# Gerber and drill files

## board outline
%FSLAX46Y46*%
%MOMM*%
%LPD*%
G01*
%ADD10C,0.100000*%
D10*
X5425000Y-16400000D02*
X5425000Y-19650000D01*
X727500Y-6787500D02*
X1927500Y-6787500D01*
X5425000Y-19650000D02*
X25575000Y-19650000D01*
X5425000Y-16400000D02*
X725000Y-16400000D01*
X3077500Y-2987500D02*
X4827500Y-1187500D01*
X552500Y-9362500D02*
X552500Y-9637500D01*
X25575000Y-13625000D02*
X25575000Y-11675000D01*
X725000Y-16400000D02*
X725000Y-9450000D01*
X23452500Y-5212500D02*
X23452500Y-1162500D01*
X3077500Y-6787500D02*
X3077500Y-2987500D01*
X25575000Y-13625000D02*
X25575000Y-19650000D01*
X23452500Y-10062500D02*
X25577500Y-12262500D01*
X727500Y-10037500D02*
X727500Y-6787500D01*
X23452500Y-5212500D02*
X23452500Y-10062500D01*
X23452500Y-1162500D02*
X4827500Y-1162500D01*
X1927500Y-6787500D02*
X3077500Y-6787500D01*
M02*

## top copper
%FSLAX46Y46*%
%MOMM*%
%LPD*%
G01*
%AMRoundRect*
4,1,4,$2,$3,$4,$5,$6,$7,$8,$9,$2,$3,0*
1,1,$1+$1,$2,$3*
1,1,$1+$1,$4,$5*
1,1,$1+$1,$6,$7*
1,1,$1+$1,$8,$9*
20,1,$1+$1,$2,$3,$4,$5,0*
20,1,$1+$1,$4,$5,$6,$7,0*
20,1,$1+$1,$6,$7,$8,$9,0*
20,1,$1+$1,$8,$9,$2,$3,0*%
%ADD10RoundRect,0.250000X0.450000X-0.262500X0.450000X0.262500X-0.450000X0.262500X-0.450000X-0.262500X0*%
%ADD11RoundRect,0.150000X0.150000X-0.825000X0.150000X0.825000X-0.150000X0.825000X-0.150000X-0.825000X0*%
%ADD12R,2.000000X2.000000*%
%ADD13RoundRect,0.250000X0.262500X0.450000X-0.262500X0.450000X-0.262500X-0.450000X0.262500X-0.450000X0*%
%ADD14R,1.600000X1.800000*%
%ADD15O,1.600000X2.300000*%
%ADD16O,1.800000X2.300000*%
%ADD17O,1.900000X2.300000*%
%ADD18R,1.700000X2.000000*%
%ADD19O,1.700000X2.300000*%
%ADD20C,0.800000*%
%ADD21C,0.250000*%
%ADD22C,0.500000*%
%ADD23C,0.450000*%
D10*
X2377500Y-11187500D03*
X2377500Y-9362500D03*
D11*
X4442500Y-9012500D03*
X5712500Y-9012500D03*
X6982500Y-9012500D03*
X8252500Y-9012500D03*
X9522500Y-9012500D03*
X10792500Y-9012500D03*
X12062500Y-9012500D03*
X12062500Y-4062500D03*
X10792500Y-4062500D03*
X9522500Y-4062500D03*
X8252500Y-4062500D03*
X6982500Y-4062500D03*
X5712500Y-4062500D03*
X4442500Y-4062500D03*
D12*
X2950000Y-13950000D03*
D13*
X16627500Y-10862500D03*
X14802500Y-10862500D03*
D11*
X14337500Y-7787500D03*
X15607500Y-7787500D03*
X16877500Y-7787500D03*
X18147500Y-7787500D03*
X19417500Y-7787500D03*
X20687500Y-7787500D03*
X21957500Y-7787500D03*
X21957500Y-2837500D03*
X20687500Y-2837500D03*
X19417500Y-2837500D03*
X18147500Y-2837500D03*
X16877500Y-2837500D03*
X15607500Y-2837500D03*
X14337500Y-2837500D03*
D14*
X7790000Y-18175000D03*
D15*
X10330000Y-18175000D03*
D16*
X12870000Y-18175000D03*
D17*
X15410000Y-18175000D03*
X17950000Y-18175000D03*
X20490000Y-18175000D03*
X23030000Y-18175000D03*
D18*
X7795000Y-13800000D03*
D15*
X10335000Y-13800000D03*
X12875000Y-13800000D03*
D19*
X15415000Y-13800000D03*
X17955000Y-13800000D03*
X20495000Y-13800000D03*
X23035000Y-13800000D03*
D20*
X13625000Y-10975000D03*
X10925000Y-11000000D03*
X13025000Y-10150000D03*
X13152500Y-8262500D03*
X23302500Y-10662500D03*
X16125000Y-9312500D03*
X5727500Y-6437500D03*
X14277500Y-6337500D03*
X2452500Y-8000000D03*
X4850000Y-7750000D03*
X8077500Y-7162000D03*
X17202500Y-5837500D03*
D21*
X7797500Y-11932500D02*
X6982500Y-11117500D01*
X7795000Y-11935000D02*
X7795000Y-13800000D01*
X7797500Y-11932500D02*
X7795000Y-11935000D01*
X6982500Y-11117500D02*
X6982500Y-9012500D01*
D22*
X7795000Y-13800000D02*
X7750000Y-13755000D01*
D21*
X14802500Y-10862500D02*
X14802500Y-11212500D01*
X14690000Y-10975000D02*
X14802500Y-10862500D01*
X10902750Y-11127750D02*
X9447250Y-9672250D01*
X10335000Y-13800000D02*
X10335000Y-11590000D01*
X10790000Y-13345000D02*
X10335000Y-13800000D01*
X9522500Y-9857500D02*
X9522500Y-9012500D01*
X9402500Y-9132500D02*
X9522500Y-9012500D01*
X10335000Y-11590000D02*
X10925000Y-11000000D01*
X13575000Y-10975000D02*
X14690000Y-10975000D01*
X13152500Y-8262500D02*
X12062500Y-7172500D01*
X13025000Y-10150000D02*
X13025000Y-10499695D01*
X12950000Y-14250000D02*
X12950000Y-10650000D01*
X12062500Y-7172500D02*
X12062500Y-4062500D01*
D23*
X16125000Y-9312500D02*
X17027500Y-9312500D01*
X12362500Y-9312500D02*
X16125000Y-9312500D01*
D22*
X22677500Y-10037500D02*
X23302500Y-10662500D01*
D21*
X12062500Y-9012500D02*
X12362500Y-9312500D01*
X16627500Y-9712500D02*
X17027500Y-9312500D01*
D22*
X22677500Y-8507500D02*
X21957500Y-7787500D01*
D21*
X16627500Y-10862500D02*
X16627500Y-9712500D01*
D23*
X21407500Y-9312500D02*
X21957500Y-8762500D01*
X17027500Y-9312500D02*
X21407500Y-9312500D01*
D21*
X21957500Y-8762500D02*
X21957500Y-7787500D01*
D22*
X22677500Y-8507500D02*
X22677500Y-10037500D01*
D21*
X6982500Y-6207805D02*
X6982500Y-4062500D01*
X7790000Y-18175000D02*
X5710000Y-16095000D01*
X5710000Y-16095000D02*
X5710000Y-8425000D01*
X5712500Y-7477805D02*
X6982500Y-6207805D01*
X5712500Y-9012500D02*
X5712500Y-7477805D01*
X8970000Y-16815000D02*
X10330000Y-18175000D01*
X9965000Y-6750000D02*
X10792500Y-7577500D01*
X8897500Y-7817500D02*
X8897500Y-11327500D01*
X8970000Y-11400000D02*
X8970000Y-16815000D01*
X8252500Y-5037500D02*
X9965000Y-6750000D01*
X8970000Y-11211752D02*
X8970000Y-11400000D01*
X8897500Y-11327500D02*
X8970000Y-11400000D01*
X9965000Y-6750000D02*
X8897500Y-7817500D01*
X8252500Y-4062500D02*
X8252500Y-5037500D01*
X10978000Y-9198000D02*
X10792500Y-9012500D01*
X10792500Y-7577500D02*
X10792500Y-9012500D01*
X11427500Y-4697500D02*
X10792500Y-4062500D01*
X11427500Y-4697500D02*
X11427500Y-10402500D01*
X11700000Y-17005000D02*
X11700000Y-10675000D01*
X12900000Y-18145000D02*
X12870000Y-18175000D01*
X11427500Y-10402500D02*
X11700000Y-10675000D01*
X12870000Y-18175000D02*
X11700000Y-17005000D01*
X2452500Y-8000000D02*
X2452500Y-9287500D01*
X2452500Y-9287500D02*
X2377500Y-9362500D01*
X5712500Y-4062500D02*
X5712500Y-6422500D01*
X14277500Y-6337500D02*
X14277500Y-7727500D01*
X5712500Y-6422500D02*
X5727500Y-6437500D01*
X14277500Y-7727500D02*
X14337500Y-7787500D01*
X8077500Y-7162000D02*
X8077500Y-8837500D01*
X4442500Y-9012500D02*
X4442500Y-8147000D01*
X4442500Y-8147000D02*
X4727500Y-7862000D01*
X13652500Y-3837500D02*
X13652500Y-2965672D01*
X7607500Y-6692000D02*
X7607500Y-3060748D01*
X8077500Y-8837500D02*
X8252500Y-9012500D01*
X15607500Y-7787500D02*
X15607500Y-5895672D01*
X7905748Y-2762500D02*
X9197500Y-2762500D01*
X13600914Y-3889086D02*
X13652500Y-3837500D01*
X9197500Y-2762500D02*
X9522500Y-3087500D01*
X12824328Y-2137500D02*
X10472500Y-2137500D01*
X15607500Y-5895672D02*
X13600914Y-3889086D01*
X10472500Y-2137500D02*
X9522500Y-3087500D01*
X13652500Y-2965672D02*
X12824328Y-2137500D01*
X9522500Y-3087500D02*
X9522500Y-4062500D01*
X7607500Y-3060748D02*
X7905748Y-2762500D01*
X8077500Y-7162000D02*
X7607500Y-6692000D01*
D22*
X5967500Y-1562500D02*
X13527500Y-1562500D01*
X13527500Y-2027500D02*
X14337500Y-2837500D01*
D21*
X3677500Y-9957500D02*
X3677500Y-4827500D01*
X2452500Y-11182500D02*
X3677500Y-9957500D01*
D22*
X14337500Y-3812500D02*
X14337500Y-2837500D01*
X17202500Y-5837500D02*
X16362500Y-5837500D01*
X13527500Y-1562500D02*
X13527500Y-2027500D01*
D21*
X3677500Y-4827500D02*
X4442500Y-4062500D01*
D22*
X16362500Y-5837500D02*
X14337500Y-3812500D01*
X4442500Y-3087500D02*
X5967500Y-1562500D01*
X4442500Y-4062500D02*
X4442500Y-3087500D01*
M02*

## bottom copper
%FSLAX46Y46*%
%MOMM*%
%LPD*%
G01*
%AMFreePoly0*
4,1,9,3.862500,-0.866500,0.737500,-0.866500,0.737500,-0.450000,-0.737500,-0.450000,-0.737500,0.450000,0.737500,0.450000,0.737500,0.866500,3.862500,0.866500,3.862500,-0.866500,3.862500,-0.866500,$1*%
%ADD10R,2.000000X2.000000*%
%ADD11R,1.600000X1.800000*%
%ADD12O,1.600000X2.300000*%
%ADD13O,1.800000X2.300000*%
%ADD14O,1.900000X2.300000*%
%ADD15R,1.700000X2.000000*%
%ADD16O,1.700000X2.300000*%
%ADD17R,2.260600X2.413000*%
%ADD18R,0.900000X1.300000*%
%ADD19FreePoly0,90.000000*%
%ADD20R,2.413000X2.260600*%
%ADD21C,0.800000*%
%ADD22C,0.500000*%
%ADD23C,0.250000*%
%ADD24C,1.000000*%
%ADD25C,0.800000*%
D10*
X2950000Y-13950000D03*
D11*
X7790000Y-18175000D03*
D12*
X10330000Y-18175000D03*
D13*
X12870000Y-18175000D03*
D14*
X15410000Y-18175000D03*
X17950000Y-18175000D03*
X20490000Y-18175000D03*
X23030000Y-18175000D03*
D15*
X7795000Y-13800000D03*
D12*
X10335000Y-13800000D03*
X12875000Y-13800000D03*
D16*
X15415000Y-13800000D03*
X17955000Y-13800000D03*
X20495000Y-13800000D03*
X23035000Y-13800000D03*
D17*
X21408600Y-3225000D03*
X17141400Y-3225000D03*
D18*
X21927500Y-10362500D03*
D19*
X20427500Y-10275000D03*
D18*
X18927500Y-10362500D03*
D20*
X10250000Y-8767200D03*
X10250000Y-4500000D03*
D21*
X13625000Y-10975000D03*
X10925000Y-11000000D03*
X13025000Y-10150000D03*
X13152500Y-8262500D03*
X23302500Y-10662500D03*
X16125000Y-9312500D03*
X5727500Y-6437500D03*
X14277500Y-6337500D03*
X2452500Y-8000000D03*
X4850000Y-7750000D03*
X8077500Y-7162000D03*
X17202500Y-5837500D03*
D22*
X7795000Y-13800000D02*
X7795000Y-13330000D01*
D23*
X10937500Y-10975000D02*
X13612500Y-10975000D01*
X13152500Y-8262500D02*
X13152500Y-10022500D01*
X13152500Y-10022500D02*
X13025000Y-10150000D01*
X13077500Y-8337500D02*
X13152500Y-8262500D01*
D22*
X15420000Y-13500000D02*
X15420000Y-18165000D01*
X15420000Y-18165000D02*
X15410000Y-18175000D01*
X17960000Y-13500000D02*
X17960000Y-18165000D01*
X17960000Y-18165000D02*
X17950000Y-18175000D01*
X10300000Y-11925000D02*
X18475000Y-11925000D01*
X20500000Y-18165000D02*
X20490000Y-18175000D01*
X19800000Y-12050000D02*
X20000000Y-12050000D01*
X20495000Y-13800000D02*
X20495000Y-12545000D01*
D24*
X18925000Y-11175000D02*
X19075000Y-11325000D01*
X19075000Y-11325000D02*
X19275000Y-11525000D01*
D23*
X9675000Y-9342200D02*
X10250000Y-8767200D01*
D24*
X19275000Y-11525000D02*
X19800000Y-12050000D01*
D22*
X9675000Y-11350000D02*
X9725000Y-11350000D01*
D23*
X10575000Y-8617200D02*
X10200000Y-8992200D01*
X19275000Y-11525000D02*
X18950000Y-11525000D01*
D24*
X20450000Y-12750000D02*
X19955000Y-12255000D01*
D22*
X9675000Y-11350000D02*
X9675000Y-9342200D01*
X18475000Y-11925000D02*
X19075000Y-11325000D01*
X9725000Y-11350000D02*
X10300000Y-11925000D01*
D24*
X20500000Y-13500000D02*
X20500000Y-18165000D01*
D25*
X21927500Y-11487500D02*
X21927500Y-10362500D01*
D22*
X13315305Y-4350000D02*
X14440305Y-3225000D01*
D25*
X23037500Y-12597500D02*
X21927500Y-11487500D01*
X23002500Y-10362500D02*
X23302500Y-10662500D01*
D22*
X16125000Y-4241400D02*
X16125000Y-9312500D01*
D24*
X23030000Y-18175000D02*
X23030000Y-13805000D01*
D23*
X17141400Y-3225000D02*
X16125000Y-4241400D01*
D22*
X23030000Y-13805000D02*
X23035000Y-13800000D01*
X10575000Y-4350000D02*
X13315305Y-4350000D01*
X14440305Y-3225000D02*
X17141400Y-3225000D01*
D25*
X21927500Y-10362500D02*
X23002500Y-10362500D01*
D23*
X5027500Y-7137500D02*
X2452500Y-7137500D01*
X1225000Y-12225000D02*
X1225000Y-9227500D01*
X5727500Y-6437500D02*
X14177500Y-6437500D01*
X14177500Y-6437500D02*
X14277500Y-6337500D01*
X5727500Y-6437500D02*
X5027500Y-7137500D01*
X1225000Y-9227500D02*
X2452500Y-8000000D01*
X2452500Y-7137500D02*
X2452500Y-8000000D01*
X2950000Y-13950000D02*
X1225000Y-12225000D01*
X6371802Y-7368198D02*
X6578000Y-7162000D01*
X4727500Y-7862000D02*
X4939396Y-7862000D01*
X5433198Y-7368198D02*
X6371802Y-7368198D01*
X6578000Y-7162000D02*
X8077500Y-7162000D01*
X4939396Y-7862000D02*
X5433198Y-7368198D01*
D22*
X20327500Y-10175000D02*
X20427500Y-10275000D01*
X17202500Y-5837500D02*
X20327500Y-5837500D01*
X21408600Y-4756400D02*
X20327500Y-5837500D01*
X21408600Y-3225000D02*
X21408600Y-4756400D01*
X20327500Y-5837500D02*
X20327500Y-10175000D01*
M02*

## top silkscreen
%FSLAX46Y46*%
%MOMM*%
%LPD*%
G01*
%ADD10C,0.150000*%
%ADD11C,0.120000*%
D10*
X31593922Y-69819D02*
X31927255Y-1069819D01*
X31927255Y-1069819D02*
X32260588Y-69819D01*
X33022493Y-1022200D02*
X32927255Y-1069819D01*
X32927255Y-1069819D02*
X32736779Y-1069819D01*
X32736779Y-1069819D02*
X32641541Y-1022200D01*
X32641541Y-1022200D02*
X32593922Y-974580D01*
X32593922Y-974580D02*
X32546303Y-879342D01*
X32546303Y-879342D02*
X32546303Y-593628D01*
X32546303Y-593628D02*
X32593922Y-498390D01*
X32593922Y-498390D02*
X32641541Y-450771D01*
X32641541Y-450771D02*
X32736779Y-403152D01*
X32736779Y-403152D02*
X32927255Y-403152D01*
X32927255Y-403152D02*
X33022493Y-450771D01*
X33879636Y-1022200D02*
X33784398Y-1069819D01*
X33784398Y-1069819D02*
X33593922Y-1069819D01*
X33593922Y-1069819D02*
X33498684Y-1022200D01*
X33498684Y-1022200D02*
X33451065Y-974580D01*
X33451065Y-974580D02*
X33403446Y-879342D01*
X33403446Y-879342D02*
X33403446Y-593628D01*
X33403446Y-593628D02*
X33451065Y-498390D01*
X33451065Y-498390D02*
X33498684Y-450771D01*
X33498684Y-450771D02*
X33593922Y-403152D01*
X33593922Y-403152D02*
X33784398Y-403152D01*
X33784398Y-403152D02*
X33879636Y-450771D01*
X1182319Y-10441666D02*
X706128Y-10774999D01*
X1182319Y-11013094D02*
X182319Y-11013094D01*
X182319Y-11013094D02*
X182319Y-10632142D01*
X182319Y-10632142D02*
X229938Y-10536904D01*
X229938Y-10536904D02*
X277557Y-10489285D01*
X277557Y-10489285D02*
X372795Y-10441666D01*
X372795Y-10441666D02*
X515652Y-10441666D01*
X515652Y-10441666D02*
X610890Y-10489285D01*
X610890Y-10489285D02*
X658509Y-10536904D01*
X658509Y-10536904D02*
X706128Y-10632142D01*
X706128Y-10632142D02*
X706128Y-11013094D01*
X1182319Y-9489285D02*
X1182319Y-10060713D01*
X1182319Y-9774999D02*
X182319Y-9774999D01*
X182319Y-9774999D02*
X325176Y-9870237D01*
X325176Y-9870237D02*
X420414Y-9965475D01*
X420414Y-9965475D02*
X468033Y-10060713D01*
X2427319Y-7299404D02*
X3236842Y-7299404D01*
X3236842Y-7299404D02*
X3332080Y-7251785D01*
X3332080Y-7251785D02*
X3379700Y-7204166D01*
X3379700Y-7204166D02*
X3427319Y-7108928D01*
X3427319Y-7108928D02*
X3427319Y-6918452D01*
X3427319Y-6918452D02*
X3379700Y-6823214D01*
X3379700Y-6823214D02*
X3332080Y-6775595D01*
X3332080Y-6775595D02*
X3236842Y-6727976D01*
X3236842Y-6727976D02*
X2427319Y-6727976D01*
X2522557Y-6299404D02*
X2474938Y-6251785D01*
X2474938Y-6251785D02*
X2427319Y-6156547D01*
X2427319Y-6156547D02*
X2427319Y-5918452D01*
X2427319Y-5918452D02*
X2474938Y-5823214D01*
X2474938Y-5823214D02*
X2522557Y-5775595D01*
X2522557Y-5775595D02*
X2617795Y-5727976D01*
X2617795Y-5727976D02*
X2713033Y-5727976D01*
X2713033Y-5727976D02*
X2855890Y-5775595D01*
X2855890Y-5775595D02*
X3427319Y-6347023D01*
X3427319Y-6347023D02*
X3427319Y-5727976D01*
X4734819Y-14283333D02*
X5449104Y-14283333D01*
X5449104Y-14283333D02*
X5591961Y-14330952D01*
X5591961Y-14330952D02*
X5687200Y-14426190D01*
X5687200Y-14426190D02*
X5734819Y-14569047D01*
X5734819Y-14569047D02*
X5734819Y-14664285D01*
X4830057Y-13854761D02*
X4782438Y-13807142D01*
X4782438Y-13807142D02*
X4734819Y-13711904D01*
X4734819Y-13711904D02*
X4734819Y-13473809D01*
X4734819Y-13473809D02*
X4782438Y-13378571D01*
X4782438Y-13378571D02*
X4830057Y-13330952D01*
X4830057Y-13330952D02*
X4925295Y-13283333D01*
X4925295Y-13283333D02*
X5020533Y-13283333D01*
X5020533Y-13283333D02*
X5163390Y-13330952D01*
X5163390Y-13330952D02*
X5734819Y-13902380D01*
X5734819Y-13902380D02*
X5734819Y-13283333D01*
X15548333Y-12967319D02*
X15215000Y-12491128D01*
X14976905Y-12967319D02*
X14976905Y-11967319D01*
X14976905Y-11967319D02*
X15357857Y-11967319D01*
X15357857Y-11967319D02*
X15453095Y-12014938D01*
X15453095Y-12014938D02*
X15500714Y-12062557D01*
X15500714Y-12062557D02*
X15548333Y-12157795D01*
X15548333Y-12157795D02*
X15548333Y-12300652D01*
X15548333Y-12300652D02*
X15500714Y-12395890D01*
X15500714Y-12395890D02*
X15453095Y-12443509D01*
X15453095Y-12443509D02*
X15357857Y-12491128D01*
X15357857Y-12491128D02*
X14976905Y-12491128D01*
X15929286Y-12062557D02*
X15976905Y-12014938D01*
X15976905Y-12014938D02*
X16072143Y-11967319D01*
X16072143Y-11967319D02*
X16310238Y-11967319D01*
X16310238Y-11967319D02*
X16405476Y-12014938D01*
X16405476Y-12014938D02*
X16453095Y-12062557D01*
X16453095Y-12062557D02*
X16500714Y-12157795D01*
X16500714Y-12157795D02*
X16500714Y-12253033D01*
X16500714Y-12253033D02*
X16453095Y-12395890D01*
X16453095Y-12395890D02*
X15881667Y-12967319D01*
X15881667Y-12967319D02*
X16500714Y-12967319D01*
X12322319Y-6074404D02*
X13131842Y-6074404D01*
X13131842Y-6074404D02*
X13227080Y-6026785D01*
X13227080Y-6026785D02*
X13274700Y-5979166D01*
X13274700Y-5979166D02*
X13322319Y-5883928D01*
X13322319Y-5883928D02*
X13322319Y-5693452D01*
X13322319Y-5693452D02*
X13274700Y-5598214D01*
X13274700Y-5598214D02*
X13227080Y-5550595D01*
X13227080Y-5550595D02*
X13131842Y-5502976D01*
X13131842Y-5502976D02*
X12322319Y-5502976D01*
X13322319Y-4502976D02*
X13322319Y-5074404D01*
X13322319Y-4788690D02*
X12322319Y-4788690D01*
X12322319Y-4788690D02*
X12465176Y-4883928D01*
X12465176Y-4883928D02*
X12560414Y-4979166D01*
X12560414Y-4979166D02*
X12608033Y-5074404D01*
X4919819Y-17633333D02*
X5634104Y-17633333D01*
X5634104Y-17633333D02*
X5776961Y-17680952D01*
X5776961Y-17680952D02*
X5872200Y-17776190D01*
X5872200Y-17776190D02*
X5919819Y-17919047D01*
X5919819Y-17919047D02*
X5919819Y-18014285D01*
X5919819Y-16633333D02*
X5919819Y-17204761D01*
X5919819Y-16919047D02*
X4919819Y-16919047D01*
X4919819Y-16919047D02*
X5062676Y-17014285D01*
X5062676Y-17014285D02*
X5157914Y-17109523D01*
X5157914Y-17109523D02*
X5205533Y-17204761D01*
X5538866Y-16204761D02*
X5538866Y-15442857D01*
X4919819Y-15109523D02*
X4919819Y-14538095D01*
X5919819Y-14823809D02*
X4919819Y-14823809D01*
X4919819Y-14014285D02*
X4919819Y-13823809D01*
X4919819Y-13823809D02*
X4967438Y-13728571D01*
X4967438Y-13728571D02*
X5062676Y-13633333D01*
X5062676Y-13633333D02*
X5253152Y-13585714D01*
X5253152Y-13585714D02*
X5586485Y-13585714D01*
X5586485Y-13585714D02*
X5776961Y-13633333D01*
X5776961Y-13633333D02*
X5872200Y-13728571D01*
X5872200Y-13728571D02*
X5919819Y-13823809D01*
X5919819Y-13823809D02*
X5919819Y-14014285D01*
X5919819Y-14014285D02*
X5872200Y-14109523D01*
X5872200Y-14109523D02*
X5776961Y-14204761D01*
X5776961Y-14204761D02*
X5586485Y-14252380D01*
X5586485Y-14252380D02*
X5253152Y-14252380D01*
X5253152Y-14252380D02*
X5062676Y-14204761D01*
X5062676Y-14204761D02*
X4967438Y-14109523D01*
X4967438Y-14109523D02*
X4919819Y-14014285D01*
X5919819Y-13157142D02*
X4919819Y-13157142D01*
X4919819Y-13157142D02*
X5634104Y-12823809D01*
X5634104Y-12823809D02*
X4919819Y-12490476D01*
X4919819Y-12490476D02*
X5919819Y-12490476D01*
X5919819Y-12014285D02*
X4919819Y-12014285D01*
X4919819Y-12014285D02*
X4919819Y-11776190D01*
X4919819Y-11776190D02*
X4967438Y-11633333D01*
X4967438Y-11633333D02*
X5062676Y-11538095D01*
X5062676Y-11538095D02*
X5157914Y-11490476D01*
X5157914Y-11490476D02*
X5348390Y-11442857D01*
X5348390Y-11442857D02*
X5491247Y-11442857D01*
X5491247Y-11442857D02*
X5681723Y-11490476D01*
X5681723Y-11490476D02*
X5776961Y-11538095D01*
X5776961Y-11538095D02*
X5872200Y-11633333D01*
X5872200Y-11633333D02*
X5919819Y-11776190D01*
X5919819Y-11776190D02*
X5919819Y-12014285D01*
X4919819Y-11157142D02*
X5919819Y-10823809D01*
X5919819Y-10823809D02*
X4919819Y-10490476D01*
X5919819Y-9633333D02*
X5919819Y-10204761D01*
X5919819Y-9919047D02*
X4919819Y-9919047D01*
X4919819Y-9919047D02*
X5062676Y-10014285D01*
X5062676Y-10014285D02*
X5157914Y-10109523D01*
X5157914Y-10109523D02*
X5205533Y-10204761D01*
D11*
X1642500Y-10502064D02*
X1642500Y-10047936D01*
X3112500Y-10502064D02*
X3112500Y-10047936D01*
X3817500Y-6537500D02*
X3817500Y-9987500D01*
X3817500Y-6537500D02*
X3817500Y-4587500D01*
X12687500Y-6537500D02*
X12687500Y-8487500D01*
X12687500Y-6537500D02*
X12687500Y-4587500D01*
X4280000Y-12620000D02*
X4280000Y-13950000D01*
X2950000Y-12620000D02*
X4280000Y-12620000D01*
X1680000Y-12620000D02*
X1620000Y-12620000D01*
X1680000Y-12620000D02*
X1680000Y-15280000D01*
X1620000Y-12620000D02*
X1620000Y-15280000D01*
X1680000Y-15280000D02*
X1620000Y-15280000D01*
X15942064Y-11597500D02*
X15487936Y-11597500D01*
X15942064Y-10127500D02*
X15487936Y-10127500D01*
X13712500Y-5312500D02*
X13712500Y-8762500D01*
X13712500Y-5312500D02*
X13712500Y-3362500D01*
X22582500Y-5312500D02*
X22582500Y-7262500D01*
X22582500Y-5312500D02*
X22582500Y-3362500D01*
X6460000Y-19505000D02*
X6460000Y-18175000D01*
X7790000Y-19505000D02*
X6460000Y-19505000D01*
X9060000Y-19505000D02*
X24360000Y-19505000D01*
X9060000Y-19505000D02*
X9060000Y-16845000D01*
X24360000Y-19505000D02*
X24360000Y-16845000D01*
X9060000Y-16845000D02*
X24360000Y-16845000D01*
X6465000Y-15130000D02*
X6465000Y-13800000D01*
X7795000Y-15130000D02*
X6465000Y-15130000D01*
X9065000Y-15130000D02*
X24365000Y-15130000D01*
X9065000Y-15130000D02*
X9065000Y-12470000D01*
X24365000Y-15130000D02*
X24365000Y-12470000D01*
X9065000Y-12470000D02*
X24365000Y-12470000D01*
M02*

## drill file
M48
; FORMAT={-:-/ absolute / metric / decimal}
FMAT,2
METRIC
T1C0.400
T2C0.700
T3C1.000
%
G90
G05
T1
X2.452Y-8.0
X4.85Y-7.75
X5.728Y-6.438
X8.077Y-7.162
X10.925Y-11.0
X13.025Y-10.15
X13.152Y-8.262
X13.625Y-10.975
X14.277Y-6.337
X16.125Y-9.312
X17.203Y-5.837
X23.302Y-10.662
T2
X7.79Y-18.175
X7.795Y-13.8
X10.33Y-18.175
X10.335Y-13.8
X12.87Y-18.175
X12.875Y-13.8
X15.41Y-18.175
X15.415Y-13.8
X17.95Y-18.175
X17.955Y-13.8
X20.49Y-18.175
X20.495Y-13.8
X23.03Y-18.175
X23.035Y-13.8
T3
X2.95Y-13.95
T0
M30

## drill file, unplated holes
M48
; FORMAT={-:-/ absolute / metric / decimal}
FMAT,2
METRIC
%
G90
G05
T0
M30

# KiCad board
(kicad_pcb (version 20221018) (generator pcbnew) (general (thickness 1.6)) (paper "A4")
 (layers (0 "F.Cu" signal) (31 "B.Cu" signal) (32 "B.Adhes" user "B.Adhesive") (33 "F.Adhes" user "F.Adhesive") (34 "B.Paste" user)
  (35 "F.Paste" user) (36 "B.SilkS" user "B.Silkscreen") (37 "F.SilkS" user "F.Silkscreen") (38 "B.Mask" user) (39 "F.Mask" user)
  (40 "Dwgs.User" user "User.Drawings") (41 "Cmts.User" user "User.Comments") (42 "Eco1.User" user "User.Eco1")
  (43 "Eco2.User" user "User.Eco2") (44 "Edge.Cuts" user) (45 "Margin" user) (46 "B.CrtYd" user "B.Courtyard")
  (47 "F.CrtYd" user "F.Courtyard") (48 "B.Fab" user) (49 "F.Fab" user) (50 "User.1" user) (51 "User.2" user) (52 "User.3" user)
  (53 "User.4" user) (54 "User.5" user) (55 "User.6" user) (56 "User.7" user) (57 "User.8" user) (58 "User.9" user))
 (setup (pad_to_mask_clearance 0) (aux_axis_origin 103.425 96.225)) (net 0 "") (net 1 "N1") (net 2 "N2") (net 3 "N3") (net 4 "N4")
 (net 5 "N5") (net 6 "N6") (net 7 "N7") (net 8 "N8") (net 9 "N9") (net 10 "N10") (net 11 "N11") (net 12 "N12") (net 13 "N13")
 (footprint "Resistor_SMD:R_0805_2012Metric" (layer "F.Cu") (at 105.8025 106.5 90)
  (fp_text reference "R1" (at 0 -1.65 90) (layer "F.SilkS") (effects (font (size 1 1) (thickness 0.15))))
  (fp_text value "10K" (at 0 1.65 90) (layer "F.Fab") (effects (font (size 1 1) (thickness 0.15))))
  (fp_line (start -0.227064 -0.735) (end 0.227064 -0.735) (stroke (width 0.12) (type solid)) (layer "F.SilkS"))
  (fp_line (start -0.227064 0.735) (end 0.227064 0.735) (stroke (width 0.12) (type solid)) (layer "F.SilkS"))
  (pad "1" smd roundrect (at -0.9125 0 90) (size 1.025 1.4) (layers "F.Cu" "F.Paste" "F.Mask") (roundrect_rratio 0.243902439) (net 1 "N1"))
  (pad "2" smd roundrect (at 0.9125 0 90) (size 1.025 1.4) (layers "F.Cu" "F.Paste" "F.Mask") (roundrect_rratio 0.243902439) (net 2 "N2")))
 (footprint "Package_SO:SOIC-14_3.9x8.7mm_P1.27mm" (layer "F.Cu") (at 111.6775 102.7625 90)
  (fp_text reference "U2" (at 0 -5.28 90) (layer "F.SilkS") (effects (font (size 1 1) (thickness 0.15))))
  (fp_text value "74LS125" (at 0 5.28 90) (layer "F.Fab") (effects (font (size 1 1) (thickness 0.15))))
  (fp_line (start 0 -4.435) (end -3.45 -4.435) (stroke (width 0.12) (type solid)) (layer "F.SilkS"))
  (fp_line (start 0 -4.435) (end 1.95 -4.435) (stroke (width 0.12) (type solid)) (layer "F.SilkS"))
  (fp_line (start 0 4.435) (end -1.95 4.435) (stroke (width 0.12) (type solid)) (layer "F.SilkS"))
  (fp_line (start 0 4.435) (end 1.95 4.435) (stroke (width 0.12) (type solid)) (layer "F.SilkS"))
  (pad "1" smd roundrect (at -2.475 -3.81 90) (size 1.95 0.6) (layers "F.Cu" "F.Paste" "F.Mask") (roundrect_rratio 0.25) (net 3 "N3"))
  (pad "2" smd roundrect (at -2.475 -2.54 90) (size 1.95 0.6) (layers "F.Cu" "F.Paste" "F.Mask") (roundrect_rratio 0.25) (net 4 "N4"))
  (pad "3" smd roundrect (at -2.475 -1.27 90) (size 1.95 0.6) (layers "F.Cu" "F.Paste" "F.Mask") (roundrect_rratio 0.25) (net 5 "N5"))
  (pad "4" smd roundrect (at -2.475 0 90) (size 1.95 0.6) (layers "F.Cu" "F.Paste" "F.Mask") (roundrect_rratio 0.25) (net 3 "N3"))
  (pad "5" smd roundrect (at -2.475 1.27 90) (size 1.95 0.6) (layers "F.Cu" "F.Paste" "F.Mask") (roundrect_rratio 0.25) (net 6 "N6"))
  (pad "6" smd roundrect (at -2.475 2.54 90) (size 1.95 0.6) (layers "F.Cu" "F.Paste" "F.Mask") (roundrect_rratio 0.25) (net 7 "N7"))
  (pad "7" smd roundrect (at -2.475 3.81 90) (size 1.95 0.6) (layers "F.Cu" "F.Paste" "F.Mask") (roundrect_rratio 0.25) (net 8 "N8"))
  (pad "8" smd roundrect (at 2.475 3.81 90) (size 1.95 0.6) (layers "F.Cu" "F.Paste" "F.Mask") (roundrect_rratio 0.25) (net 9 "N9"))
  (pad "9" smd roundrect (at 2.475 2.54 90) (size 1.95 0.6) (layers "F.Cu" "F.Paste" "F.Mask") (roundrect_rratio 0.25) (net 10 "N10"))
  (pad "10" smd roundrect (at 2.475 1.27 90) (size 1.95 0.6) (layers "F.Cu" "F.Paste" "F.Mask") (roundrect_rratio 0.25) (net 3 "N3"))
  (pad "11" smd roundrect (at 2.475 0 90) (size 1.95 0.6) (layers "F.Cu" "F.Paste" "F.Mask") (roundrect_rratio 0.25) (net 7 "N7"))
  (pad "12" smd roundrect (at 2.475 -1.27 90) (size 1.95 0.6) (layers "F.Cu" "F.Paste" "F.Mask") (roundrect_rratio 0.25) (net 4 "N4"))
  (pad "13" smd roundrect (at 2.475 -2.54 90) (size 1.95 0.6) (layers "F.Cu" "F.Paste" "F.Mask") (roundrect_rratio 0.25) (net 2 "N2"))
  (pad "14" smd roundrect (at 2.475 -3.81 90) (size 1.95 0.6) (layers "F.Cu" "F.Paste" "F.Mask") (roundrect_rratio 0.25) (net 1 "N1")))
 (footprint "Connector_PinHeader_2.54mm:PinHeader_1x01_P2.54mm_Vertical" (layer "F.Cu") (at 106.375 110.175 -90)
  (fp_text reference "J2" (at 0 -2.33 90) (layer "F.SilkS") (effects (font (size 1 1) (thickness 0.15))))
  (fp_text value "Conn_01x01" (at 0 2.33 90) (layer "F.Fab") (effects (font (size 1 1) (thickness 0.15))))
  (fp_line (start -1.33 -1.33) (end 0 -1.33) (stroke (width 0.12) (type solid)) (layer "F.SilkS"))
  (fp_line (start -1.33 0) (end -1.33 -1.33) (stroke (width 0.12) (type solid)) (layer "F.SilkS"))
  (fp_line (start -1.33 1.27) (end -1.33 1.33) (stroke (width 0.12) (type solid)) (layer "F.SilkS"))
  (fp_line (start -1.33 1.27) (end 1.33 1.27) (stroke (width 0.12) (type solid)) (layer "F.SilkS"))
  (fp_line (start -1.33 1.33) (end 1.33 1.33) (stroke (width 0.12) (type solid)) (layer "F.SilkS"))
  (fp_line (start 1.33 1.27) (end 1.33 1.33) (stroke (width 0.12) (type solid)) (layer "F.SilkS"))
  (pad "1" thru_hole rect (at 0 0 270) (size 2 2) (drill 1) (layers "*.Cu" "*.Mask") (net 2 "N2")))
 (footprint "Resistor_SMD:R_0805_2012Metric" (layer "F.Cu") (at 119.14 107.0875 180)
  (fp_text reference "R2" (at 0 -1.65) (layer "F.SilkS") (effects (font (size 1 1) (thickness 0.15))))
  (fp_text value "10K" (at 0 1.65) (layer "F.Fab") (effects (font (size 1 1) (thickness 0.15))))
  (fp_line (start -0.227064 -0.735) (end 0.227064 -0.735) (stroke (width 0.12) (type solid)) (layer "F.SilkS"))
  (fp_line (start -0.227064 0.735) (end 0.227064 0.735) (stroke (width 0.12) (type solid)) (layer "F.SilkS"))
  (pad "1" smd roundrect (at -0.9125 0 180) (size 1.025 1.4) (layers "F.Cu" "F.Paste" "F.Mask") (roundrect_rratio 0.243902439) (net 8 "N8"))
  (pad "2" smd roundrect (at 0.9125 0 180) (size 1.025 1.4) (layers "F.Cu" "F.Paste" "F.Mask") (roundrect_rratio 0.243902439) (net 6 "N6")))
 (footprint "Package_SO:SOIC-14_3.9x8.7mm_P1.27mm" (layer "F.Cu") (at 121.5725 101.5375 90)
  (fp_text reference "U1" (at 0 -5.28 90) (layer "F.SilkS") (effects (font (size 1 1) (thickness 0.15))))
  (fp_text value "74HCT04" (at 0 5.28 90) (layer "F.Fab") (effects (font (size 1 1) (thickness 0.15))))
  (fp_line (start 0 -4.435) (end -3.45 -4.435) (stroke (width 0.12) (type solid)) (layer "F.SilkS"))
  (fp_line (start 0 -4.435) (end 1.95 -4.435) (stroke (width 0.12) (type solid)) (layer "F.SilkS"))
  (fp_line (start 0 4.435) (end -1.95 4.435) (stroke (width 0.12) (type solid)) (layer "F.SilkS"))
  (fp_line (start 0 4.435) (end 1.95 4.435) (stroke (width 0.12) (type solid)) (layer "F.SilkS"))
  (pad "1" smd roundrect (at -2.475 -3.81 90) (size 1.95 0.6) (layers "F.Cu" "F.Paste" "F.Mask") (roundrect_rratio 0.25) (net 2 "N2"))
  (pad "2" smd roundrect (at -2.475 -2.54 90) (size 1.95 0.6) (layers "F.Cu" "F.Paste" "F.Mask") (roundrect_rratio 0.25) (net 3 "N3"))
  (pad "3" smd roundrect (at -2.475 -1.27 90) (size 1.95 0.6) (layers "F.Cu" "F.Paste" "F.Mask") (roundrect_rratio 0.25))
  (pad "4" smd roundrect (at -2.475 0 90) (size 1.95 0.6) (layers "F.Cu" "F.Paste" "F.Mask") (roundrect_rratio 0.25))
  (pad "5" smd roundrect (at -2.475 1.27 90) (size 1.95 0.6) (layers "F.Cu" "F.Paste" "F.Mask") (roundrect_rratio 0.25))
  (pad "6" smd roundrect (at -2.475 2.54 90) (size 1.95 0.6) (layers "F.Cu" "F.Paste" "F.Mask") (roundrect_rratio 0.25))
  (pad "7" smd roundrect (at -2.475 3.81 90) (size 1.95 0.6) (layers "F.Cu" "F.Paste" "F.Mask") (roundrect_rratio 0.25) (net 8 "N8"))
  (pad "8" smd roundrect (at 2.475 3.81 90) (size 1.95 0.6) (layers "F.Cu" "F.Paste" "F.Mask") (roundrect_rratio 0.25))
  (pad "9" smd roundrect (at 2.475 2.54 90) (size 1.95 0.6) (layers "F.Cu" "F.Paste" "F.Mask") (roundrect_rratio 0.25))
  (pad "10" smd roundrect (at 2.475 1.27 90) (size 1.95 0.6) (layers "F.Cu" "F.Paste" "F.Mask") (roundrect_rratio 0.25))
  (pad "11" smd roundrect (at 2.475 0 90) (size 1.95 0.6) (layers "F.Cu" "F.Paste" "F.Mask") (roundrect_rratio 0.25))
  (pad "12" smd roundrect (at 2.475 -1.27 90) (size 1.95 0.6) (layers "F.Cu" "F.Paste" "F.Mask") (roundrect_rratio 0.25))
  (pad "13" smd roundrect (at 2.475 -2.54 90) (size 1.95 0.6) (layers "F.Cu" "F.Paste" "F.Mask") (roundrect_rratio 0.25))
  (pad "14" smd roundrect (at 2.475 -3.81 90) (size 1.95 0.6) (layers "F.Cu" "F.Paste" "F.Mask") (roundrect_rratio 0.25) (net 1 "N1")))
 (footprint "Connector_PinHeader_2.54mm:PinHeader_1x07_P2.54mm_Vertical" (layer "F.Cu") (at 111.215 114.4 90)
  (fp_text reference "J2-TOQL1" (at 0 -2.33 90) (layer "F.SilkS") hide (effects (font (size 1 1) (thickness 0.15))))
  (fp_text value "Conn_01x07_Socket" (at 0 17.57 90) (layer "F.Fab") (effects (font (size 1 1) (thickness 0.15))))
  (fp_line (start -1.33 -1.33) (end 0 -1.33) (stroke (width 0.12) (type solid)) (layer "F.SilkS"))
  (fp_line (start -1.33 0) (end -1.33 -1.33) (stroke (width 0.12) (type solid)) (layer "F.SilkS"))
  (fp_line (start -1.33 1.27) (end -1.33 16.57) (stroke (width 0.12) (type solid)) (layer "F.SilkS"))
  (fp_line (start -1.33 1.27) (end 1.33 1.27) (stroke (width 0.12) (type solid)) (layer "F.SilkS"))
  (fp_line (start -1.33 16.57) (end 1.33 16.57) (stroke (width 0.12) (type solid)) (layer "F.SilkS"))
  (fp_line (start 1.33 1.27) (end 1.33 16.57) (stroke (width 0.12) (type solid)) (layer "F.SilkS"))
  (pad "1" thru_hole rect (at 0 0 90) (size 1.8 1.6) (drill 0.7) (layers "*.Cu" "*.Mask") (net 4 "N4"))
  (pad "2" thru_hole oval (at 0 2.54 90) (size 2.3 1.6) (drill 0.7) (layers "*.Cu" "*.Mask") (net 7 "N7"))
  (pad "3" thru_hole oval (at 0 5.08 90) (size 2.3 1.8) (drill 0.7) (layers "*.Cu" "*.Mask") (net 10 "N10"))
  (pad "4" thru_hole oval (at 0 7.62 90) (size 2.3 1.9) (drill 0.7) (layers "*.Cu" "*.Mask") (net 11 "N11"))
  (pad "5" thru_hole oval (at 0 10.16 90) (size 2.3 1.9) (drill 0.7) (layers "*.Cu" "*.Mask") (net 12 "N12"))
  (pad "6" thru_hole oval (at 0 12.7 90) (size 2.3 1.9) (drill 0.7) (layers "*.Cu" "*.Mask") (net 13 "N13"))
  (pad "7" thru_hole oval (at 0 15.24 90) (size 2.3 1.9) (drill 0.7) (layers "*.Cu" "*.Mask") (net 8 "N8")))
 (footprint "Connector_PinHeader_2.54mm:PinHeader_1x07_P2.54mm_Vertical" (layer "F.Cu") (at 111.22 110.025 90)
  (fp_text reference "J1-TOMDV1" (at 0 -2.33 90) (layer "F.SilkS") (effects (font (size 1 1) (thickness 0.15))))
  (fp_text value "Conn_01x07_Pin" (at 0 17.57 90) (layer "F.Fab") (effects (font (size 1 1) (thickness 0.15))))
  (fp_line (start -1.33 -1.33) (end 0 -1.33) (stroke (width 0.12) (type solid)) (layer "F.SilkS"))
  (fp_line (start -1.33 0) (end -1.33 -1.33) (stroke (width 0.12) (type solid)) (layer "F.SilkS"))
  (fp_line (start -1.33 1.27) (end -1.33 16.57) (stroke (width 0.12) (type solid)) (layer "F.SilkS"))
  (fp_line (start -1.33 1.27) (end 1.33 1.27) (stroke (width 0.12) (type solid)) (layer "F.SilkS"))
  (fp_line (start -1.33 16.57) (end 1.33 16.57) (stroke (width 0.12) (type solid)) (layer "F.SilkS"))
  (fp_line (start 1.33 1.27) (end 1.33 16.57) (stroke (width 0.12) (type solid)) (layer "F.SilkS"))
  (pad "1" thru_hole rect (at 0 0 90) (size 2 1.7) (drill 0.7) (layers "*.Cu" "*.Mask") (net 5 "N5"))
  (pad "2" thru_hole oval (at 0 2.54 90) (size 2.3 1.6) (drill 0.7) (layers "*.Cu" "*.Mask") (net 6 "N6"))
  (pad "3" thru_hole oval (at 0 5.08 90) (size 2.3 1.6) (drill 0.7) (layers "*.Cu" "*.Mask") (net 9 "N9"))
  (pad "4" thru_hole oval (at 0 7.62 90) (size 2.3 1.7) (drill 0.7) (layers "*.Cu" "*.Mask") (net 11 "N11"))
  (pad "5" thru_hole oval (at 0 10.16 90) (size 2.3 1.7) (drill 0.7) (layers "*.Cu" "*.Mask") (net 12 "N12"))
  (pad "6" thru_hole oval (at 0 12.7 90) (size 2.3 1.7) (drill 0.7) (layers "*.Cu" "*.Mask") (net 13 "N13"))
  (pad "7" thru_hole oval (at 0 15.24 90) (size 2.3 1.7) (drill 0.7) (layers "*.Cu" "*.Mask") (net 8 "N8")))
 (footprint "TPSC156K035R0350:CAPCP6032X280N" (layer "B.Cu") (at 122.7 99.45 180)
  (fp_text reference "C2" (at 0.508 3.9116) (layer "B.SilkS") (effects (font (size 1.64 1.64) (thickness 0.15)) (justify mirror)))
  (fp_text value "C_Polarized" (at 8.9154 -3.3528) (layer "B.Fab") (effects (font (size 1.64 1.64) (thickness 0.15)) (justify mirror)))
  (pad "1" smd rect (at -2.1336 0 90) (size 2.413 2.2606) (layers "B.Cu" "B.Paste" "B.Mask") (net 1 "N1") (solder_mask_margin 0.102))
  (pad "2" smd rect (at 2.1336 0 90) (size 2.413 2.2606) (layers "B.Cu" "B.Paste" "B.Mask") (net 8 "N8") (solder_mask_margin 0.102)))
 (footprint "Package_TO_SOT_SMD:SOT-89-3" (layer "B.Cu") (at 123.8525 104.6375 90)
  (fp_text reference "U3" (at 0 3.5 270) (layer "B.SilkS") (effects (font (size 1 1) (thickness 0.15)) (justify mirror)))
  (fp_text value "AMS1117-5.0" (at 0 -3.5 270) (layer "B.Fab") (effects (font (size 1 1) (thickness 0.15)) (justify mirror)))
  (pad "1" smd rect (at -1.95 1.5 90) (size 1.3 0.9) (layers "B.Cu" "B.Paste" "B.Mask") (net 8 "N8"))
  (pad "2" smd custom (at -1.8625 0 90) (size 1.475 0.9) (layers "B.Cu" "B.Paste" "B.Mask") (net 1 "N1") (zone_connect 2)
   (options (clearance outline) (anchor rect)) (primitives))
  (pad "3" smd rect (at -1.95 -1.5 90) (size 1.3 0.9) (layers "B.Cu" "B.Paste" "B.Mask") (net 13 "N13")))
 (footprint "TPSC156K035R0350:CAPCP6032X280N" (layer "B.Cu") (at 113.675 102.8586 90)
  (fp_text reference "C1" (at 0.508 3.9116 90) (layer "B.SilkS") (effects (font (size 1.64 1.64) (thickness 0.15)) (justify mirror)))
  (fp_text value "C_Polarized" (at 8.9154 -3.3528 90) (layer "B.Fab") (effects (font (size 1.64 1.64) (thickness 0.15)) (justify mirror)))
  (pad "1" smd rect (at -2.1336 0) (size 2.413 2.2606) (layers "B.Cu" "B.Paste" "B.Mask") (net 13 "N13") (solder_mask_margin 0.102))
  (pad "2" smd rect (at 2.1336 0) (size 2.413 2.2606) (layers "B.Cu" "B.Paste" "B.Mask") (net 8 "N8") (solder_mask_margin 0.102)))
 (gr_line (start 108.85 112.625) (end 108.85 115.875) (stroke (width 0.1) (type default)) (layer "Edge.Cuts"))
 (gr_line (start 104.1525 103.0125) (end 105.3525 103.0125) (stroke (width 0.1) (type default)) (layer "Edge.Cuts"))
 (gr_line (start 108.85 115.875) (end 129 115.875) (stroke (width 0.1) (type default)) (layer "Edge.Cuts"))
 (gr_line (start 108.85 112.625) (end 104.15 112.625) (stroke (width 0.1) (type default)) (layer "Edge.Cuts"))
 (gr_line (start 106.5025 99.2125) (end 108.2525 97.4125) (stroke (width 0.1) (type default)) (layer "Edge.Cuts"))
 (gr_line (start 103.9775 105.5875) (end 103.9775 105.8625) (stroke (width 0.1) (type default)) (layer "Edge.Cuts"))
 (gr_line (start 129 109.85) (end 129 107.9) (stroke (width 0.1) (type default)) (layer "Edge.Cuts"))
 (gr_line (start 104.15 112.625) (end 104.15 105.675) (stroke (width 0.1) (type default)) (layer "Edge.Cuts"))
 (gr_line (start 126.8775 101.4375) (end 126.8775 97.3875) (stroke (width 0.1) (type default)) (layer "Edge.Cuts"))
 (gr_line (start 106.5025 103.0125) (end 106.5025 99.2125) (stroke (width 0.1) (type default)) (layer "Edge.Cuts"))
 (gr_line (start 129 109.85) (end 129 115.875) (stroke (width 0.1) (type default)) (layer "Edge.Cuts"))
 (gr_line (start 126.8775 106.2875) (end 129.0025 108.4875) (stroke (width 0.1) (type default)) (layer "Edge.Cuts"))
 (gr_line (start 104.1525 106.2625) (end 104.1525 103.0125) (stroke (width 0.1) (type default)) (layer "Edge.Cuts"))
 (gr_line (start 126.8775 101.4375) (end 126.8775 106.2875) (stroke (width 0.1) (type default)) (layer "Edge.Cuts"))
 (gr_line (start 126.8775 97.3875) (end 108.2525 97.3875) (stroke (width 0.1) (type default)) (layer "Edge.Cuts"))
 (gr_line (start 105.3525 103.0125) (end 106.5025 103.0125) (stroke (width 0.1) (type default)) (layer "Edge.Cuts"))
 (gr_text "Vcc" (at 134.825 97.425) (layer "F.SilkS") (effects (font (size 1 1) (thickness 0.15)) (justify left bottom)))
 (segment (start 111.2225 108.1575) (end 110.4075 107.3425) (width 0.25) (layer "F.Cu") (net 5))
 (segment (start 111.22 108.16) (end 111.22 110.025) (width 0.25) (layer "F.Cu") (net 5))
 (segment (start 111.2225 108.1575) (end 111.22 108.16) (width 0.25) (layer "F.Cu") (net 5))
 (segment (start 110.4075 107.3425) (end 110.4075 105.2375) (width 0.25) (layer "F.Cu") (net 5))
 (segment (start 111.22 110.025) (end 111.175 109.98) (width 0.5) (layer "F.Cu") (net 5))
 (segment (start 111.22 110.025) (end 111.22 109.555) (width 0.5) (layer "B.Cu") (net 5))
 (segment (start 118.2275 107.0875) (end 118.2275 107.4375) (width 0.25) (layer "F.Cu") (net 6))
 (segment (start 118.115 107.2) (end 118.2275 107.0875) (width 0.25) (layer "F.Cu") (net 6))
 (segment (start 114.32775 107.35275) (end 112.87225 105.89725) (width 0.25) (layer "F.Cu") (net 6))
 (segment (start 113.76 110.025) (end 113.76 107.815) (width 0.25) (layer "F.Cu") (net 6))
 (segment (start 114.215 109.57) (end 113.76 110.025) (width 0.25) (layer "F.Cu") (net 6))
 (segment (start 112.9475 106.0825) (end 112.9475 105.2375) (width 0.25) (layer "F.Cu") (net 6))
 (segment (start 112.8275 105.3575) (end 112.9475 105.2375) (width 0.25) (layer "F.Cu") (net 6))
 (segment (start 113.76 107.815) (end 114.35 107.225) (width 0.25) (layer "F.Cu") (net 6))
 (segment (start 117 107.2) (end 118.115 107.2) (width 0.25) (layer "F.Cu") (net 6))
 (via (at 117.05 107.2) (size 0.8) (drill 0.4) (layers "F.Cu" "B.Cu") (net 6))
 (via (at 114.35 107.225) (size 0.8) (drill 0.4) (layers "F.Cu" "B.Cu") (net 6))
 (segment (start 114.3625 107.2) (end 117.0375 107.2) (width 0.25) (layer "B.Cu") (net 6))
 (segment (start 116.5775 104.4875) (end 115.4875 103.3975) (width 0.25) (layer "F.Cu") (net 9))
 (segment (start 116.45 106.375) (end 116.45 106.724695) (width 0.25) (layer "F.Cu") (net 9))
 (segment (start 116.375 110.475) (end 116.375 106.875) (width 0.25) (layer "F.Cu") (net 9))
 (segment (start 115.4875 103.3975) (end 115.4875 100.2875) (width 0.25) (layer "F.Cu") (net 9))
 (via (at 116.45 106.375) (size 0.8) (drill 0.4) (layers "F.Cu" "B.Cu") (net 9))
 (via (at 116.5775 104.4875) (size 0.8) (drill 0.4) (layers "F.Cu" "B.Cu") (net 9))
 (segment (start 116.5775 104.4875) (end 116.5775 106.2475) (width 0.25) (layer "B.Cu") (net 9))
 (segment (start 116.5775 106.2475) (end 116.45 106.375) (width 0.25) (layer "B.Cu") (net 9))
 (segment (start 116.5025 104.5625) (end 116.5775 104.4875) (width 0.25) (layer "B.Cu") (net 9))
 (segment (start 118.845 109.725) (end 118.845 114.39) (width 0.5) (layer "B.Cu") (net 11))
 (segment (start 118.845 114.39) (end 118.835 114.4) (width 0.5) (layer "B.Cu") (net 11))
 (segment (start 121.385 109.725) (end 121.385 114.39) (width 0.5) (layer "B.Cu") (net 12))
 (segment (start 121.385 114.39) (end 121.375 114.4) (width 0.5) (layer "B.Cu") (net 12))
 (segment (start 113.725 108.15) (end 121.9 108.15) (width 0.5) (layer "B.Cu") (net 13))
 (segment (start 123.925 114.39) (end 123.915 114.4) (width 0.5) (layer "B.Cu") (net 13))
 (segment (start 123.225 108.275) (end 123.425 108.275) (width 0.5) (layer "B.Cu") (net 13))
 (segment (start 123.92 110.025) (end 123.92 108.77) (width 0.5) (layer "B.Cu") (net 13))
 (segment (start 122.35 107.4) (end 122.5 107.55) (width 1) (layer "B.Cu") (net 13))
 (segment (start 122.5 107.55) (end 122.7 107.75) (width 1) (layer "B.Cu") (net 13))
 (segment (start 113.1 105.5672) (end 113.675 104.9922) (width 0.25) (layer "B.Cu") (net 13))
 (segment (start 122.7 107.75) (end 123.225 108.275) (width 1) (layer "B.Cu") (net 13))
 (segment (start 113.1 107.575) (end 113.15 107.575) (width 0.5) (layer "B.Cu") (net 13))
 (segment (start 114 104.8422) (end 113.625 105.2172) (width 0.25) (layer "B.Cu") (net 13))
 (segment (start 122.7 107.75) (end 122.375 107.75) (width 0.25) (layer "B.Cu") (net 13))
 (segment (start 123.875 108.975) (end 123.38 108.48) (width 1) (layer "B.Cu") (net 13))
 (segment (start 113.1 107.575) (end 113.1 105.5672) (width 0.5) (layer "B.Cu") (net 13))
 (segment (start 121.9 108.15) (end 122.5 107.55) (width 0.5) (layer "B.Cu") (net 13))
 (segment (start 113.15 107.575) (end 113.725 108.15) (width 0.5) (layer "B.Cu") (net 13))
 (segment (start 123.925 109.725) (end 123.925 114.39) (width 1) (layer "B.Cu") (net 13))
 (segment (start 119.55 105.5375) (end 120.4525 105.5375) (width 0.45) (layer "F.Cu") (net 8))
 (segment (start 115.7875 105.5375) (end 119.55 105.5375) (width 0.45) (layer "F.Cu") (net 8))
 (segment (start 126.1025 106.2625) (end 126.7275 106.8875) (width 0.5) (layer "F.Cu") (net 8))
 (segment (start 115.4875 105.2375) (end 115.7875 105.5375) (width 0.25) (layer "F.Cu") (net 8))
 (segment (start 120.0525 105.9375) (end 120.4525 105.5375) (width 0.25) (layer "F.Cu") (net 8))
 (segment (start 126.1025 104.7325) (end 125.3825 104.0125) (width 0.5) (layer "F.Cu") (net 8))
 (segment (start 120.0525 107.0875) (end 120.0525 105.9375) (width 0.25) (layer "F.Cu") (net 8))
 (segment (start 124.8325 105.5375) (end 125.3825 104.9875) (width 0.45) (layer "F.Cu") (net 8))
 (segment (start 120.4525 105.5375) (end 124.8325 105.5375) (width 0.45) (layer "F.Cu") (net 8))
 (segment (start 125.3825 104.9875) (end 125.3825 104.0125) (width 0.25) (layer "F.Cu") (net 8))
 (segment (start 126.1025 104.7325) (end 126.1025 106.2625) (width 0.5) (layer "F.Cu") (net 8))
 (via (at 126.7275 106.8875) (size 0.8) (drill 0.4) (layers "F.Cu" "B.Cu") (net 8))
 (via (at 119.55 105.5375) (size 0.8) (drill 0.4) (layers "F.Cu" "B.Cu") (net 8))
 (segment (start 125.3525 107.7125) (end 125.3525 106.5875) (width 0.8) (layer "B.Cu") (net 8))
 (segment (start 116.740305 100.575) (end 117.865305 99.45) (width 0.5) (layer "B.Cu") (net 8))
 (segment (start 126.4625 108.8225) (end 125.3525 107.7125) (width 0.8) (layer "B.Cu") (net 8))
 (segment (start 126.4275 106.5875) (end 126.7275 106.8875) (width 0.8) (layer "B.Cu") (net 8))
 (segment (start 119.55 100.4664) (end 119.55 105.5375) (width 0.5) (layer "B.Cu") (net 8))
 (segment (start 126.455 114.4) (end 126.455 110.03) (width 1) (layer "B.Cu") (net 8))
 (segment (start 120.5664 99.45) (end 119.55 100.4664) (width 0.25) (layer "B.Cu") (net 8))
 (segment (start 126.455 110.03) (end 126.46 110.025) (width 0.5) (layer "B.Cu") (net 8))
 (segment (start 114 100.575) (end 116.740305 100.575) (width 0.5) (layer "B.Cu") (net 8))
 (segment (start 117.865305 99.45) (end 120.5664 99.45) (width 0.5) (layer "B.Cu") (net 8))
 (segment (start 125.3525 106.5875) (end 126.4275 106.5875) (width 0.8) (layer "B.Cu") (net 8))
 (segment (start 110.4075 102.432805) (end 110.4075 100.2875) (width 0.25) (layer "F.Cu") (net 4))
 (segment (start 111.215 114.4) (end 109.135 112.32) (width 0.25) (layer "F.Cu") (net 4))
 (segment (start 109.135 112.32) (end 109.135 104.65) (width 0.25) (layer "F.Cu") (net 4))
 (segment (start 109.1375 103.702805) (end 110.4075 102.432805) (width 0.25) (layer "F.Cu") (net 4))
 (segment (start 109.1375 105.2375) (end 109.1375 103.702805) (width 0.25) (layer "F.Cu") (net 4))
 (segment (start 112.395 113.04) (end 113.755 114.4) (width 0.25) (layer "F.Cu") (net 7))
 (segment (start 113.39 102.975) (end 114.2175 103.8025) (width 0.25) (layer "F.Cu") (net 7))
 (segment (start 112.3225 104.0425) (end 112.3225 107.5525) (width 0.25) (layer "F.Cu") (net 7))
 (segment (start 112.395 107.625) (end 112.395 113.04) (width 0.25) (layer "F.Cu") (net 7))
 (segment (start 111.6775 101.2625) (end 113.39 102.975) (width 0.25) (layer "F.Cu") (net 7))
 (segment (start 112.395 107.436752) (end 112.395 107.625) (width 0.25) (layer "F.Cu") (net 7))
 (segment (start 112.3225 107.5525) (end 112.395 107.625) (width 0.25) (layer "F.Cu") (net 7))
 (segment (start 113.39 102.975) (end 112.3225 104.0425) (width 0.25) (layer "F.Cu") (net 7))
 (segment (start 111.6775 100.2875) (end 111.6775 101.2625) (width 0.25) (layer "F.Cu") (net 7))
 (segment (start 114.403 105.423) (end 114.2175 105.2375) (width 0.25) (layer "F.Cu") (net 7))
 (segment (start 114.2175 103.8025) (end 114.2175 105.2375) (width 0.25) (layer "F.Cu") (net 7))
 (segment (start 114.8525 100.9225) (end 114.2175 100.2875) (width 0.25) (layer "F.Cu") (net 10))
 (segment (start 114.8525 100.9225) (end 114.8525 106.6275) (width 0.25) (layer "F.Cu") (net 10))
 (segment (start 115.125 113.23) (end 115.125 106.9) (width 0.25) (layer "F.Cu") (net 10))
 (segment (start 116.325 114.37) (end 116.295 114.4) (width 0.25) (layer "F.Cu") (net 10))
 (segment (start 114.8525 106.6275) (end 115.125 106.9) (width 0.25) (layer "F.Cu") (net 10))
 (segment (start 116.295 114.4) (end 115.125 113.23) (width 0.25) (layer "F.Cu") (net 10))
 (segment (start 105.8775 104.225) (end 105.8775 105.5125) (width 0.25) (layer "F.Cu") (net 2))
 (segment (start 105.8775 105.5125) (end 105.8025 105.5875) (width 0.25) (layer "F.Cu") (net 2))
 (segment (start 109.1375 100.2875) (end 109.1375 102.6475) (width 0.25) (layer "F.Cu") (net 2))
 (segment (start 117.7025 102.5625) (end 117.7025 103.9525) (width 0.25) (layer "F.Cu") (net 2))
 (segment (start 109.1375 102.6475) (end 109.1525 102.6625) (width 0.25) (layer "F.Cu") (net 2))
 (segment (start 117.7025 103.9525) (end 117.7625 104.0125) (width 0.25) (layer "F.Cu") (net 2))
 (via (at 109.1525 102.6625) (size 0.8) (drill 0.4) (layers "F.Cu" "B.Cu") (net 2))
 (via (at 117.7025 102.5625) (size 0.8) (drill 0.4) (layers "F.Cu" "B.Cu") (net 2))
 (via (at 105.8775 104.225) (size 0.8) (drill 0.4) (layers "F.Cu" "B.Cu") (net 2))
 (segment (start 108.4525 103.3625) (end 105.8775 103.3625) (width 0.25) (layer "B.Cu") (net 2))
 (segment (start 104.65 108.45) (end 104.65 105.4525) (width 0.25) (layer "B.Cu") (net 2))
 (segment (start 109.1525 102.6625) (end 117.6025 102.6625) (width 0.25) (layer "B.Cu") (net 2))
 (segment (start 117.6025 102.6625) (end 117.7025 102.5625) (width 0.25) (layer "B.Cu") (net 2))
 (segment (start 109.1525 102.6625) (end 108.4525 103.3625) (width 0.25) (layer "B.Cu") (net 2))
 (segment (start 104.65 105.4525) (end 105.8775 104.225) (width 0.25) (layer "B.Cu") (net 2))
 (segment (start 105.8775 103.3625) (end 105.8775 104.225) (width 0.25) (layer "B.Cu") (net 2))
 (segment (start 106.375 110.175) (end 104.65 108.45) (width 0.25) (layer "B.Cu") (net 2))
 (segment (start 111.5025 103.387) (end 111.5025 105.0625) (width 0.25) (layer "F.Cu") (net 3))
 (segment (start 107.8675 105.2375) (end 107.8675 104.372) (width 0.25) (layer "F.Cu") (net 3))
 (segment (start 107.8675 104.372) (end 108.1525 104.087) (width 0.25) (layer "F.Cu") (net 3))
 (segment (start 117.0775 100.0625) (end 117.0775 99.190672) (width 0.25) (layer "F.Cu") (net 3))
 (segment (start 111.0325 102.917) (end 111.0325 99.285748) (width 0.25) (layer "F.Cu") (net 3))
 (segment (start 111.5025 105.0625) (end 111.6775 105.2375) (width 0.25) (layer "F.Cu") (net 3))
 (segment (start 119.0325 104.0125) (end 119.0325 102.120672) (width 0.25) (layer "F.Cu") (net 3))
 (segment (start 111.330748 98.9875) (end 112.6225 98.9875) (width 0.25) (layer "F.Cu") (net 3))
 (segment (start 117.025914 100.114086) (end 117.0775 100.0625) (width 0.25) (layer "F.Cu") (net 3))
 (segment (start 112.6225 98.9875) (end 112.9475 99.3125) (width 0.25) (layer "F.Cu") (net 3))
 (segment (start 116.249328 98.3625) (end 113.8975 98.3625) (width 0.25) (layer "F.Cu") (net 3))
 (segment (start 119.0325 102.120672) (end 117.025914 100.114086) (width 0.25) (layer "F.Cu") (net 3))
 (segment (start 113.8975 98.3625) (end 112.9475 99.3125) (width 0.25) (layer "F.Cu") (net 3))
 (segment (start 117.0775 99.190672) (end 116.249328 98.3625) (width 0.25) (layer "F.Cu") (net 3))
 (segment (start 112.9475 99.3125) (end 112.9475 100.2875) (width 0.25) (layer "F.Cu") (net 3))
 (segment (start 111.0325 99.285748) (end 111.330748 98.9875) (width 0.25) (layer "F.Cu") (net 3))
 (segment (start 111.5025 103.387) (end 111.0325 102.917) (width 0.25) (layer "F.Cu") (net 3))
 (via (at 108.275 103.975) (size 0.8) (drill 0.4) (layers "F.Cu" "B.Cu") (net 3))
 (via (at 111.5025 103.387) (size 0.8) (drill 0.4) (layers "F.Cu" "B.Cu") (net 3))
 (segment (start 109.796802 103.593198) (end 110.003 103.387) (width 0.25) (layer "B.Cu") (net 3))
 (segment (start 108.1525 104.087) (end 108.364396 104.087) (width 0.25) (layer "B.Cu") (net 3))
 (segment (start 108.858198 103.593198) (end 109.796802 103.593198) (width 0.25) (layer "B.Cu") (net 3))
 (segment (start 110.003 103.387) (end 111.5025 103.387) (width 0.25) (layer "B.Cu") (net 3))
 (segment (start 108.364396 104.087) (end 108.858198 103.593198) (width 0.25) (layer "B.Cu") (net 3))
 (segment (start 109.3925 97.7875) (end 116.9525 97.7875) (width 0.5) (layer "F.Cu") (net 1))
 (segment (start 116.9525 98.2525) (end 117.7625 99.0625) (width 0.5) (layer "F.Cu") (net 1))
 (segment (start 107.1025 106.1825) (end 107.1025 101.0525) (width 0.25) (layer "F.Cu") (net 1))
 (segment (start 105.8775 107.4075) (end 107.1025 106.1825) (width 0.25) (layer "F.Cu") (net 1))
 (segment (start 117.7625 100.0375) (end 117.7625 99.0625) (width 0.5) (layer "F.Cu") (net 1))
 (segment (start 120.6275 102.0625) (end 119.7875 102.0625) (width 0.5) (layer "F.Cu") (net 1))
 (segment (start 116.9525 97.7875) (end 116.9525 98.2525) (width 0.5) (layer "F.Cu") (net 1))
 (segment (start 107.1025 101.0525) (end 107.8675 100.2875) (width 0.25) (layer "F.Cu") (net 1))
 (segment (start 119.7875 102.0625) (end 117.7625 100.0375) (width 0.5) (layer "F.Cu") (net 1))
 (segment (start 107.8675 99.3125) (end 109.3925 97.7875) (width 0.5) (layer "F.Cu") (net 1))
 (segment (start 107.8675 100.2875) (end 107.8675 99.3125) (width 0.5) (layer "F.Cu") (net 1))
 (via (at 120.6275 102.0625) (size 0.8) (drill 0.4) (layers "F.Cu" "B.Cu") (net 1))
 (segment (start 123.7525 106.4) (end 123.8525 106.5) (width 0.5) (layer "B.Cu") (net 1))
 (segment (start 120.6275 102.0625) (end 123.7525 102.0625) (width 0.5) (layer "B.Cu") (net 1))
 (segment (start 124.8336 100.9814) (end 123.7525 102.0625) (width 0.5) (layer "B.Cu") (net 1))
 (segment (start 124.8336 99.45) (end 124.8336 100.9814) (width 0.5) (layer "B.Cu") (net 1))
 (segment (start 123.7525 102.0625) (end 123.7525 106.4) (width 0.5) (layer "B.Cu") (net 1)))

